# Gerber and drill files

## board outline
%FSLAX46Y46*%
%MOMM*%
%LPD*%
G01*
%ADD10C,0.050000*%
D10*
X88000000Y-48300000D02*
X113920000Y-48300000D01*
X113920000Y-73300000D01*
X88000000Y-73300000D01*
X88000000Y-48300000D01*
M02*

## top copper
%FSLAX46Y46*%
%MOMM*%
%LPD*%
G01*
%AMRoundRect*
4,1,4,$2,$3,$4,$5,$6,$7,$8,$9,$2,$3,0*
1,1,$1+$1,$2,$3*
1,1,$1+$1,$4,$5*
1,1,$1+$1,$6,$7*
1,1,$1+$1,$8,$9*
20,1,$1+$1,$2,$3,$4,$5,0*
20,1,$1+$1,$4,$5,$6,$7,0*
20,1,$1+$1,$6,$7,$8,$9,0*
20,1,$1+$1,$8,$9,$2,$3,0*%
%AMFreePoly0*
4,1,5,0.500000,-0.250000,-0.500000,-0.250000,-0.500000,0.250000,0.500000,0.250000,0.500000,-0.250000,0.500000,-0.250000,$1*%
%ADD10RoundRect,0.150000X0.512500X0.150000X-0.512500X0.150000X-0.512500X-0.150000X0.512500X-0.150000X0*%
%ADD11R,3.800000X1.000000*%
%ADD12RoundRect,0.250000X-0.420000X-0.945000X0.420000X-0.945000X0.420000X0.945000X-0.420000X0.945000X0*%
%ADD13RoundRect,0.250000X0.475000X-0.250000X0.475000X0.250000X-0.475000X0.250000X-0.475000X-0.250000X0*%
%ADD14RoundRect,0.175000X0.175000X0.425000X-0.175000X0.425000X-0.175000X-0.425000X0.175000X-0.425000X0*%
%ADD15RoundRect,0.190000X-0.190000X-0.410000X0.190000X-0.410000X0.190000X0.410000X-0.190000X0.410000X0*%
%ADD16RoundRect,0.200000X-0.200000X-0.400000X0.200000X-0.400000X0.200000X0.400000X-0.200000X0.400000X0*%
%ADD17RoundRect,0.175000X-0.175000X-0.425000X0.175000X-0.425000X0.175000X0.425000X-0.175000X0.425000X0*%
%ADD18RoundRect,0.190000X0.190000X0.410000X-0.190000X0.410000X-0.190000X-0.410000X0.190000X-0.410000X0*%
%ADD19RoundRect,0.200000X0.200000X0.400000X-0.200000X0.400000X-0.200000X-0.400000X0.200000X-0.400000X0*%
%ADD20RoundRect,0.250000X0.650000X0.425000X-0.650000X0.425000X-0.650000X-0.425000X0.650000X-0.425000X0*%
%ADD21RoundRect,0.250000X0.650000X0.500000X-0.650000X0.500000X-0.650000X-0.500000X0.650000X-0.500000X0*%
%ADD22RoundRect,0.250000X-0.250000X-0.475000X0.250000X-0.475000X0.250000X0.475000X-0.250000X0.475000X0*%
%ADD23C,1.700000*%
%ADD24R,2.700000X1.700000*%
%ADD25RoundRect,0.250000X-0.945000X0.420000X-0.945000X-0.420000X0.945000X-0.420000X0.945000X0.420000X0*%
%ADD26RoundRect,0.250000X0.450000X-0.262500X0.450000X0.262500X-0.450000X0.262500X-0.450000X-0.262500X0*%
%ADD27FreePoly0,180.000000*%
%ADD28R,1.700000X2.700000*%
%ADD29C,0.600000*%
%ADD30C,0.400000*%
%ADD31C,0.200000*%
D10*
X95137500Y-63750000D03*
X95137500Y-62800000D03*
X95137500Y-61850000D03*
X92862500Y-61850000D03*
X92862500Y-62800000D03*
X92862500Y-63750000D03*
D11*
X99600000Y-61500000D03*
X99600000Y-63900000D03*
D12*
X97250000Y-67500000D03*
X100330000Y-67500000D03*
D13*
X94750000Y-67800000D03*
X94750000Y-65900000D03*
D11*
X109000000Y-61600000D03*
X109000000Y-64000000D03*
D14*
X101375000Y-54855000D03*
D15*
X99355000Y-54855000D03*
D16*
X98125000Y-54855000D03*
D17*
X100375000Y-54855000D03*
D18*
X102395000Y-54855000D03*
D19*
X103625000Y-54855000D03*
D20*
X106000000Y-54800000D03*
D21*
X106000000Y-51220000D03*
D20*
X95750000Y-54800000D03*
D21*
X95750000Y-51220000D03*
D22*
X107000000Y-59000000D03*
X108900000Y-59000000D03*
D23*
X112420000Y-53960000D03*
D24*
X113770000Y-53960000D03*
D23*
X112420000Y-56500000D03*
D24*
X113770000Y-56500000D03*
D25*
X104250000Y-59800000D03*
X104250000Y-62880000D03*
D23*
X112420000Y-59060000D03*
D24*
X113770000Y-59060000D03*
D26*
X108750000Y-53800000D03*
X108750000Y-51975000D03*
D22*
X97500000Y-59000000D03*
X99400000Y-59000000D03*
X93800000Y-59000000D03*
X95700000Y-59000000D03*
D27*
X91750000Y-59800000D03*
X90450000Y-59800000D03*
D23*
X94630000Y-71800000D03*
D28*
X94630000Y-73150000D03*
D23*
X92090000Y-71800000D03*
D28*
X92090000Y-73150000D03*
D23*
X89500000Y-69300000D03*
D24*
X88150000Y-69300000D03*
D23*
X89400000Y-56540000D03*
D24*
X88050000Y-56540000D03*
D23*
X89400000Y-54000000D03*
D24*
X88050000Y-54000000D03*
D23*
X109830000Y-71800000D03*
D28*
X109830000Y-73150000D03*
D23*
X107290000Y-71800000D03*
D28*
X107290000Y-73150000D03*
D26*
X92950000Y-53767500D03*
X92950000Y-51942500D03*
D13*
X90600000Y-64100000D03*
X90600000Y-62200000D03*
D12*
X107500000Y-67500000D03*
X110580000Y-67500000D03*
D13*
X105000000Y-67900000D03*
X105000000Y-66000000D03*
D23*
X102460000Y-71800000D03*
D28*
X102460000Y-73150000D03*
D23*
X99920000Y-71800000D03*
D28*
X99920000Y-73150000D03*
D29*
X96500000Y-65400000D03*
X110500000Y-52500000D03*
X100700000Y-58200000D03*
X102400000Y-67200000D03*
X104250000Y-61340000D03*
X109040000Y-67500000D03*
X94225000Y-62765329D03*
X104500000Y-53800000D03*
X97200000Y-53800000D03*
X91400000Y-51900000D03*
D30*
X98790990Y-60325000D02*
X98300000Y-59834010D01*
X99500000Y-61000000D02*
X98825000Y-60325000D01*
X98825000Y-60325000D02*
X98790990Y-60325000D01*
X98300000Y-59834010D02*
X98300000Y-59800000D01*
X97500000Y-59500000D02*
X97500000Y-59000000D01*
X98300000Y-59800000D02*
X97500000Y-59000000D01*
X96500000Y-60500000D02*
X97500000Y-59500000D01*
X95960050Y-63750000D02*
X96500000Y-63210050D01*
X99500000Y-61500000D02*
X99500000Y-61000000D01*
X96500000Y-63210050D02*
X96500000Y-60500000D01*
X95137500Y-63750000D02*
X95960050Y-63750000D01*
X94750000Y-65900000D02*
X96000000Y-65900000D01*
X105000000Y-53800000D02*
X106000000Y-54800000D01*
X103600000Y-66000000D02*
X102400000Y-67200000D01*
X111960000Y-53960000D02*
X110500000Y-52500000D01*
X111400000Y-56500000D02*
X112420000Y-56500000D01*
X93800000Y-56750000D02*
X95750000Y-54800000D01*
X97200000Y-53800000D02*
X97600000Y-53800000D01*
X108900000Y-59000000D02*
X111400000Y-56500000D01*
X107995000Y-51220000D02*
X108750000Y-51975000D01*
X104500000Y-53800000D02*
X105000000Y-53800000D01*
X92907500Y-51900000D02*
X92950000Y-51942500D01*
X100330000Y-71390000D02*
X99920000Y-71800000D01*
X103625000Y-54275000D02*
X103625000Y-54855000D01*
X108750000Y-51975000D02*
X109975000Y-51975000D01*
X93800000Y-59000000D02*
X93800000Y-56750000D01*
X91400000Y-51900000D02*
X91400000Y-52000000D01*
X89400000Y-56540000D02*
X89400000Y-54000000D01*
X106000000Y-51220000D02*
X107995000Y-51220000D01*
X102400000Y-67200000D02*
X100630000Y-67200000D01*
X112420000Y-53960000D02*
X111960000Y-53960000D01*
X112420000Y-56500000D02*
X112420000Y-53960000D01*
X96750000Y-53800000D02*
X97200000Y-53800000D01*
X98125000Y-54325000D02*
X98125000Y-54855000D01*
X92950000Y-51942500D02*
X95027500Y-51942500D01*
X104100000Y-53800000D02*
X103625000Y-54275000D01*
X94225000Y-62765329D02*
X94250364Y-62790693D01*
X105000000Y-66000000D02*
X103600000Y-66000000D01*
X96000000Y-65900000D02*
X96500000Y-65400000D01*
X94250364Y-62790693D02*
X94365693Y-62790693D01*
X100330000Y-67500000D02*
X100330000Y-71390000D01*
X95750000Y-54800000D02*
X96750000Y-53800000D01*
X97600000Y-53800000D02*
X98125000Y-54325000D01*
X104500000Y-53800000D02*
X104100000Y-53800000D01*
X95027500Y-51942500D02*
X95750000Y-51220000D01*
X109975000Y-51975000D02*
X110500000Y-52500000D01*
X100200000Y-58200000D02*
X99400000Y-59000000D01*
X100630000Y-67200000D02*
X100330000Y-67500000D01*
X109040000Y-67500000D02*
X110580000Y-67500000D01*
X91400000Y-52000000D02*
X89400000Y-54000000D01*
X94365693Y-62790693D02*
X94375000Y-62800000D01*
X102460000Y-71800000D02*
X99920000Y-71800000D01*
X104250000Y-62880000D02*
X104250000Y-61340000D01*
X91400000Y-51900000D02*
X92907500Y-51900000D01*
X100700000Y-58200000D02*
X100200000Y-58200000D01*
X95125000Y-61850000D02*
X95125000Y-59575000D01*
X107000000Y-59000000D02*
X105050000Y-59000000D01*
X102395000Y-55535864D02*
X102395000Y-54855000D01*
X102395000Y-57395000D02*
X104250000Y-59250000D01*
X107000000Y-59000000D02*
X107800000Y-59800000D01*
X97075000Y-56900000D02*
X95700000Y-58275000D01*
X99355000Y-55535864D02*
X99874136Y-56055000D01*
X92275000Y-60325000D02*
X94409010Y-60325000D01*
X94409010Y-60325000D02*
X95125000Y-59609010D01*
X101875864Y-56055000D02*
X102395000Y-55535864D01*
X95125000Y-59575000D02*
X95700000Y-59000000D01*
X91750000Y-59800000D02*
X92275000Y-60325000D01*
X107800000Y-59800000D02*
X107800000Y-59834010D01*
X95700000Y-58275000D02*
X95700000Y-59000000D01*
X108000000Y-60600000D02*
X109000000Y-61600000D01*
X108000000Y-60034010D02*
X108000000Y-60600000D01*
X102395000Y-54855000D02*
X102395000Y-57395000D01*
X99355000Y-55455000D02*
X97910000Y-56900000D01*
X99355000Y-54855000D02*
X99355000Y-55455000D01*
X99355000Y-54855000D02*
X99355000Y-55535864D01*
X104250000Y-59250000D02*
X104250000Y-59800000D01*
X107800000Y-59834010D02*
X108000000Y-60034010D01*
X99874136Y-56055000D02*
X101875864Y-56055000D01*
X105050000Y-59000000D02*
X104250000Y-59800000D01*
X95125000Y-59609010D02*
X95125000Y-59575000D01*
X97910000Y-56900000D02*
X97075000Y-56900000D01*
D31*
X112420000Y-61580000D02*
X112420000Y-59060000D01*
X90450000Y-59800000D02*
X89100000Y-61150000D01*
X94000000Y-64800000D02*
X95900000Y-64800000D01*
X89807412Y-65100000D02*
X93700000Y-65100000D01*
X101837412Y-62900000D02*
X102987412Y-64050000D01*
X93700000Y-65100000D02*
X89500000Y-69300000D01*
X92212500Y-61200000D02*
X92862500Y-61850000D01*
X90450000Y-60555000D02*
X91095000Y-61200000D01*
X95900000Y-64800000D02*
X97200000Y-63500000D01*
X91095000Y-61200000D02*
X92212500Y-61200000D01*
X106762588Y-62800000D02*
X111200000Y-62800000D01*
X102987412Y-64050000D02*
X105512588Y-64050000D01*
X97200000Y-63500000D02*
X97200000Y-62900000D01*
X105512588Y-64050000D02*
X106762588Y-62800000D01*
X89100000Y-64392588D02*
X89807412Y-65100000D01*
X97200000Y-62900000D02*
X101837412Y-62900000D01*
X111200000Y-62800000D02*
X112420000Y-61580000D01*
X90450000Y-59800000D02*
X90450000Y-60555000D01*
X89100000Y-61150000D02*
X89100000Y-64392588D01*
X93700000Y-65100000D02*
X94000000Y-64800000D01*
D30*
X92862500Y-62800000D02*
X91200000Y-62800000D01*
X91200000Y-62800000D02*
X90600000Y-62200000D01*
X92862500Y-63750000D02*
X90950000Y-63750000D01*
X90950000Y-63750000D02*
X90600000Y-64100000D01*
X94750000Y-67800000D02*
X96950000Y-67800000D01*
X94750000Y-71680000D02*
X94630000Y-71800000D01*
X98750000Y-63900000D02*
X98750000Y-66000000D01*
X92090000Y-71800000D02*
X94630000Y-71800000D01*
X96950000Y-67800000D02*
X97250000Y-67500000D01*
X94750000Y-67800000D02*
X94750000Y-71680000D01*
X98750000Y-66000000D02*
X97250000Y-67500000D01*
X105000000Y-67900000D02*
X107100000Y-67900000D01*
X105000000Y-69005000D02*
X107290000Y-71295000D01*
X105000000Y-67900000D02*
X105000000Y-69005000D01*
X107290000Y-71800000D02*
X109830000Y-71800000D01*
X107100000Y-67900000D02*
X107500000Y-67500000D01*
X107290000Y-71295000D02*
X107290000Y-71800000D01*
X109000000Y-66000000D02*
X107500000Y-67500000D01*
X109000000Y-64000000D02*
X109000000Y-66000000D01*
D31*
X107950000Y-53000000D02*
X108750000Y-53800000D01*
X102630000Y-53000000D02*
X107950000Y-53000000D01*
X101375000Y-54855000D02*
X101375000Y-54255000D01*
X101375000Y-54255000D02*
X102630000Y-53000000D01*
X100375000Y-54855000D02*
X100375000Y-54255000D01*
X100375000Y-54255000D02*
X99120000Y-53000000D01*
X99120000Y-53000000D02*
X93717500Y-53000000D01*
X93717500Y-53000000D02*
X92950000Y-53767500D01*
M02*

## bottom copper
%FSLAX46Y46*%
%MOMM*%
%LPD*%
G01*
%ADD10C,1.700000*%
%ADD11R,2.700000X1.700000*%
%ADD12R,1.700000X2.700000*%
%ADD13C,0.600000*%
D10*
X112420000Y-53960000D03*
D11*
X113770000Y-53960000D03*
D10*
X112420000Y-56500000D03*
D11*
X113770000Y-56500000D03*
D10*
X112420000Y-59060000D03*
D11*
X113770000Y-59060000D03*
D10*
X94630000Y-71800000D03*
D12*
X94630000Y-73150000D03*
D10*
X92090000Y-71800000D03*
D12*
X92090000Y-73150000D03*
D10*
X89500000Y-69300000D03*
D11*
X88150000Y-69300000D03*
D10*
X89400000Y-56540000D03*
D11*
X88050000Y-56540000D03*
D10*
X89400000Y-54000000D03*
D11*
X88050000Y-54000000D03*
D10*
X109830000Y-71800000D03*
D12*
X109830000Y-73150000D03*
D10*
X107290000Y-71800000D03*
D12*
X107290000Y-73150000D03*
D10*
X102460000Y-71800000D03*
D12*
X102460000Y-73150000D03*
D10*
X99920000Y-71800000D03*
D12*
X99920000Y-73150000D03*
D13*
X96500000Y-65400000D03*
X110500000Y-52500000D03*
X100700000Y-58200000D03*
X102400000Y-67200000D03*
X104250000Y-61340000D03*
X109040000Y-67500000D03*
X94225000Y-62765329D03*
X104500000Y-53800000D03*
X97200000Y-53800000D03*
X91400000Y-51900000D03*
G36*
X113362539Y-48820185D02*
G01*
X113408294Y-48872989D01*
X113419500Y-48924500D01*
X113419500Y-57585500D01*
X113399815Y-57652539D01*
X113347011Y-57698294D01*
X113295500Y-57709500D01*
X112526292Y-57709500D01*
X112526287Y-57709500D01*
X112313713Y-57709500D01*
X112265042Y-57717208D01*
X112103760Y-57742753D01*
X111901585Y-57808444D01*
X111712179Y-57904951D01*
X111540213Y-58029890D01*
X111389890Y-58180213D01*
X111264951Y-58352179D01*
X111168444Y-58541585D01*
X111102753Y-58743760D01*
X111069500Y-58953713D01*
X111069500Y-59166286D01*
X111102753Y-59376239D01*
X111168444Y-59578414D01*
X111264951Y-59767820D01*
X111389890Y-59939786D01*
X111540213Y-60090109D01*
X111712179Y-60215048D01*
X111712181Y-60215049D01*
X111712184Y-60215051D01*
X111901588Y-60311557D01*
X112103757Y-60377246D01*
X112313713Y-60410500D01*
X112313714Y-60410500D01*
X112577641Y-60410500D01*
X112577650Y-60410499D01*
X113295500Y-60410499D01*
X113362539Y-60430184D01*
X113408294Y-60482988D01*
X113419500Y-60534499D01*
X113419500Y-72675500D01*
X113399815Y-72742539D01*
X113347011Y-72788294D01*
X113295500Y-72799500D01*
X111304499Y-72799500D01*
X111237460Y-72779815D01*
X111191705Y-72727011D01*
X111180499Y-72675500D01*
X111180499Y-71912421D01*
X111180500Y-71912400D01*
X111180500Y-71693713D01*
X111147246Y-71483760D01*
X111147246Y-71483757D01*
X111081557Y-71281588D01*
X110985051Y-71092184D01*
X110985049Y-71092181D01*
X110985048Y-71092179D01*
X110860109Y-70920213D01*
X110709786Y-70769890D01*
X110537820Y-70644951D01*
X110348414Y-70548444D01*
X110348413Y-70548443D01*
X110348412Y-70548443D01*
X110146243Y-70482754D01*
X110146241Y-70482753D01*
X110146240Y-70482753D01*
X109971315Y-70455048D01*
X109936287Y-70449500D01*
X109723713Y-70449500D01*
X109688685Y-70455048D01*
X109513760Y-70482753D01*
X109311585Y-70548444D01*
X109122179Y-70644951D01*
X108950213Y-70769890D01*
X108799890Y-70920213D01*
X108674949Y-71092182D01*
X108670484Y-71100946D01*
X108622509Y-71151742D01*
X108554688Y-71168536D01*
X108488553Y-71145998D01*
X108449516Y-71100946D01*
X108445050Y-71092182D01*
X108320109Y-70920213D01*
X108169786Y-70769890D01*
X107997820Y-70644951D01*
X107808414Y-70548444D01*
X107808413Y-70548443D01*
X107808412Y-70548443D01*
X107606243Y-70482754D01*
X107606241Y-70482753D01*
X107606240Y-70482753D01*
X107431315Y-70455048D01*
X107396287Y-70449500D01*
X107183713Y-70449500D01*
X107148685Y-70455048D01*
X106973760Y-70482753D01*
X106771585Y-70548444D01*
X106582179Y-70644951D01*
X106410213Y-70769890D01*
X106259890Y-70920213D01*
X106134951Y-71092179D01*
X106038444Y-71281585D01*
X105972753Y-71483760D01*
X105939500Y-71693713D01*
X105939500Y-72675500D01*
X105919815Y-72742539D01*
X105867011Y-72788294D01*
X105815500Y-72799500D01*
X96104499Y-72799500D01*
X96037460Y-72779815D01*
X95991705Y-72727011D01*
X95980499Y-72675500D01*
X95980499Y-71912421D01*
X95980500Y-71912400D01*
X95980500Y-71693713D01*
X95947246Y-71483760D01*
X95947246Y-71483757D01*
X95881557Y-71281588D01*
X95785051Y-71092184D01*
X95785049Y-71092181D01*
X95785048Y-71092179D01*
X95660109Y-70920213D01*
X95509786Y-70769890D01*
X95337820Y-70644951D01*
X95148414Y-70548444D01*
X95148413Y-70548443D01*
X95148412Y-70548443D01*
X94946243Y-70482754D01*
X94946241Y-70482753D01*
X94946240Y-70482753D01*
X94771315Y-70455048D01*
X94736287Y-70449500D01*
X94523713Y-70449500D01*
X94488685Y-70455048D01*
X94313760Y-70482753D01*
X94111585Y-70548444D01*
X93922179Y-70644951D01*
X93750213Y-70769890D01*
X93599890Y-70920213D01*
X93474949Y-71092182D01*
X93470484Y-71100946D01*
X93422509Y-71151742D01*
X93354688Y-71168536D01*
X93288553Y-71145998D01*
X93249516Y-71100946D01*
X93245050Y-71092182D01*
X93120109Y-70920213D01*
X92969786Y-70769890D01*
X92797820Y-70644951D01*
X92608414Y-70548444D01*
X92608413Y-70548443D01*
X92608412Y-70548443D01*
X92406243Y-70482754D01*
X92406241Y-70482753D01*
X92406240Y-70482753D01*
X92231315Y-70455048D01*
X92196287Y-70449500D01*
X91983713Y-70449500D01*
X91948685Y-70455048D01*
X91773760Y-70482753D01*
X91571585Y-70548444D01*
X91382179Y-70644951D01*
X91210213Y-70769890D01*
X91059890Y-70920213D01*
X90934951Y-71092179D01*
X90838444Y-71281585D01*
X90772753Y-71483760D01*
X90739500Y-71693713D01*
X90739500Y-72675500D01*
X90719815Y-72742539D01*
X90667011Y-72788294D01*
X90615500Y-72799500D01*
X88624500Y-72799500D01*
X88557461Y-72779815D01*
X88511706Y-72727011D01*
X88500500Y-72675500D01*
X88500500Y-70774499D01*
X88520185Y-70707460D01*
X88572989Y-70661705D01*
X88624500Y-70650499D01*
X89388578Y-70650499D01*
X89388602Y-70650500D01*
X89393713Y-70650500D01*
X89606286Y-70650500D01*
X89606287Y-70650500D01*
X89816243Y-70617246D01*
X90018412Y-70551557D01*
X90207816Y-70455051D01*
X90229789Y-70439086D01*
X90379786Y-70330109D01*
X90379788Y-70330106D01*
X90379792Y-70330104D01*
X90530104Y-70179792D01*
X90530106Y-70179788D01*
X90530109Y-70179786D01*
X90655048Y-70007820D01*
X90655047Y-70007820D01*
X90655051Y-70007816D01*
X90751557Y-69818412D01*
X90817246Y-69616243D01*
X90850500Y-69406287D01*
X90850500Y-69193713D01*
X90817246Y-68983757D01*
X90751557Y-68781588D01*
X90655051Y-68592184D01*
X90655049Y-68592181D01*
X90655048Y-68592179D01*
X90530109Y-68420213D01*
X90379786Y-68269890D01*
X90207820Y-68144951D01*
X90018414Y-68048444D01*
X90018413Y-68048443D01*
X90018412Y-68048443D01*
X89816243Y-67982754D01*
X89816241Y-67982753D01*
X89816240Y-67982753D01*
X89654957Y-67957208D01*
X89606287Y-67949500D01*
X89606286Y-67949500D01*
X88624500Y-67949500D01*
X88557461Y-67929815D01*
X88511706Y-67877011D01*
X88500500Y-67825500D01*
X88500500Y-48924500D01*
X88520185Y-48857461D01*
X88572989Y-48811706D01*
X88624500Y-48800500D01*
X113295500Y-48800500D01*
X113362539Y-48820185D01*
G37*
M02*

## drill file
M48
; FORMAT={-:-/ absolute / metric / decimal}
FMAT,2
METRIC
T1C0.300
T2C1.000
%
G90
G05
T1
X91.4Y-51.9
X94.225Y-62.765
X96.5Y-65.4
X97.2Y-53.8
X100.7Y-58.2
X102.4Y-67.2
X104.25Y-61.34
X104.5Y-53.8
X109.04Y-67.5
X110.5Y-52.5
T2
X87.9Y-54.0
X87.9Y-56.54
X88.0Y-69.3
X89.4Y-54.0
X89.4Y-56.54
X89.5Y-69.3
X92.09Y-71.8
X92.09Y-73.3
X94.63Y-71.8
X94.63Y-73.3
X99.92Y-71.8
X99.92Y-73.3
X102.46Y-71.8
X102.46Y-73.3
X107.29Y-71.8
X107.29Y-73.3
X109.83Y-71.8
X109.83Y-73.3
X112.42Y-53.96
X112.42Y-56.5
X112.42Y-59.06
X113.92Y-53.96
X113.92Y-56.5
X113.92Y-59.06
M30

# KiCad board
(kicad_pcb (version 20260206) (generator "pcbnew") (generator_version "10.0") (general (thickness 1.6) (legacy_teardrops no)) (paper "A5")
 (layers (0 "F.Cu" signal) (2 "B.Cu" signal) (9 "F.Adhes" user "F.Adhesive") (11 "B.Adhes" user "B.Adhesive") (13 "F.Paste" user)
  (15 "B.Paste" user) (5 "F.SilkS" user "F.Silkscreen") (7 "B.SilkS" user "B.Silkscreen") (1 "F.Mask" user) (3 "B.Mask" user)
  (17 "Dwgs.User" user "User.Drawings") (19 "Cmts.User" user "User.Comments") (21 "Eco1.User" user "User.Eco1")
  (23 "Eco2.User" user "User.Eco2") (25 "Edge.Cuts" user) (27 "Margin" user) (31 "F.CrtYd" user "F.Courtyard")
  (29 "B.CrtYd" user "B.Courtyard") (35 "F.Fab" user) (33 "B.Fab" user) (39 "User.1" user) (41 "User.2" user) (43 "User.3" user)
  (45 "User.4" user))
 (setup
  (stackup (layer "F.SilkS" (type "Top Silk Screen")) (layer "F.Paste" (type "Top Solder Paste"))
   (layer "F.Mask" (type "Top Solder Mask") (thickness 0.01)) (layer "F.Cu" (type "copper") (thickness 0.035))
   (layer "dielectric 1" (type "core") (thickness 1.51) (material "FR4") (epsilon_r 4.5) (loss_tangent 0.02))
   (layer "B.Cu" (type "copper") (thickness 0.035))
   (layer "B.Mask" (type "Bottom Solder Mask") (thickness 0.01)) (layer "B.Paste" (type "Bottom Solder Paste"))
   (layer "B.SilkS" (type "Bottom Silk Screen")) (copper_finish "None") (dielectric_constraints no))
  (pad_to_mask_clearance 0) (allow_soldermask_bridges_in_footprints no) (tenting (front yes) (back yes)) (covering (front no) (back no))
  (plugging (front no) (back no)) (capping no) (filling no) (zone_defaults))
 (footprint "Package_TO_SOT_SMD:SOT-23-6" (layer "F.Cu") (at 94 62.8 180)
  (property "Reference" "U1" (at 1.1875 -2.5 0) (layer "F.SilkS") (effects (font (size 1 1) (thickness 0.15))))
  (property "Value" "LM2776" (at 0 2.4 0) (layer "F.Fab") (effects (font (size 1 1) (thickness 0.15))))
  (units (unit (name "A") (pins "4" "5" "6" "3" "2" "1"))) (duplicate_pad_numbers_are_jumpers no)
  (pad "1" smd roundrect (at -1.1375 -0.95 180) (size 1.325 0.6) (layers "F.Cu" "F.Mask" "F.Paste") (roundrect_rratio 0.25) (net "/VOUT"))
  (pad "2" smd roundrect (at -1.1375 0 180) (size 1.325 0.6) (layers "F.Cu" "F.Mask" "F.Paste") (roundrect_rratio 0.25) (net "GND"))
  (pad "3" smd roundrect (at -1.1375 0.95 180) (size 1.325 0.6) (layers "F.Cu" "F.Mask" "F.Paste") (roundrect_rratio 0.25) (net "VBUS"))
  (pad "4" smd roundrect (at 1.1375 0.95 180) (size 1.325 0.6) (layers "F.Cu" "F.Mask" "F.Paste") (roundrect_rratio 0.25) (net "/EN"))
  (pad "5" smd roundrect (at 1.1375 0 180) (size 1.325 0.6) (layers "F.Cu" "F.Mask" "F.Paste") (roundrect_rratio 0.25) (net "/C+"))
  (pad "6" smd roundrect (at 1.1375 -0.95 180) (size 1.325 0.6) (layers "F.Cu" "F.Mask" "F.Paste") (roundrect_rratio 0.25) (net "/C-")))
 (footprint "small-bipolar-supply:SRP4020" (layer "F.Cu") (at 99.6 62.7)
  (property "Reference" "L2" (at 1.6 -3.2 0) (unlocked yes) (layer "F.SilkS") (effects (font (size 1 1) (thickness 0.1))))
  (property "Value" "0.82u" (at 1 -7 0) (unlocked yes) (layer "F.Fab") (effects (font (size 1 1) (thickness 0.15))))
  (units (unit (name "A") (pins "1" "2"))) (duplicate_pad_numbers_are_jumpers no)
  (pad "1" smd rect (at 0 -1.2) (size 3.8 1) (layers "F.Cu" "F.Mask" "F.Paste") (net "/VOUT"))
  (pad "2" smd rect (at 0 1.2) (size 3.8 1) (layers "F.Cu" "F.Mask" "F.Paste") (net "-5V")))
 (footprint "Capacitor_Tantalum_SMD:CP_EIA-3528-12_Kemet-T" (layer "F.Cu") (at 98.79 67.5)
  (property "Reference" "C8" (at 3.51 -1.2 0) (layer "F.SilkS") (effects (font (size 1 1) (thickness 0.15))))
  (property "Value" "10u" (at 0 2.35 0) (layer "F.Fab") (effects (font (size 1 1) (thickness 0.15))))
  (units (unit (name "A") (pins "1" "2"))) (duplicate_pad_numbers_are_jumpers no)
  (pad "1" smd roundrect (at -1.54 0) (size 1.34 2.39) (layers "F.Cu" "F.Mask" "F.Paste") (roundrect_rratio 0.186567) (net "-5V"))
  (pad "2" smd roundrect (at 1.54 0) (size 1.34 2.39) (layers "F.Cu" "F.Mask" "F.Paste") (roundrect_rratio 0.186567) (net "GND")))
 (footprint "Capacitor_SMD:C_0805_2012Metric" (layer "F.Cu") (at 94.75 66.85 90)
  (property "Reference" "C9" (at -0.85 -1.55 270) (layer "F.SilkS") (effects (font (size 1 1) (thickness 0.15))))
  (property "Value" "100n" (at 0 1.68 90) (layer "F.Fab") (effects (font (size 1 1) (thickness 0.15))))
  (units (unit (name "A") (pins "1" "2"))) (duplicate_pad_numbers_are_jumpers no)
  (pad "1" smd roundrect (at -0.95 0 90) (size 1 1.45) (layers "F.Cu" "F.Mask" "F.Paste") (roundrect_rratio 0.25) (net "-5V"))
  (pad "2" smd roundrect (at 0.95 0 90) (size 1 1.45) (layers "F.Cu" "F.Mask" "F.Paste") (roundrect_rratio 0.25) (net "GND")))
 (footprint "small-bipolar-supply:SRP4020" (layer "F.Cu") (at 109 62.8)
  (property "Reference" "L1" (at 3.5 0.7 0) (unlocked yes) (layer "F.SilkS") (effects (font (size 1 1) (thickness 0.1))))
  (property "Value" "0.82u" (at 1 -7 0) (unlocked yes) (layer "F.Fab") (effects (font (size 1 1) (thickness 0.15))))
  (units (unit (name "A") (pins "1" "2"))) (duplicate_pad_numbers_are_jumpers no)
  (pad "1" smd rect (at 0 -1.2) (size 3.8 1) (layers "F.Cu" "F.Mask" "F.Paste") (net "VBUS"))
  (pad "2" smd rect (at 0 1.2) (size 3.8 1) (layers "F.Cu" "F.Mask" "F.Paste") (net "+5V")))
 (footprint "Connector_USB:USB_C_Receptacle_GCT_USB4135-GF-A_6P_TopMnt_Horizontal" (layer "F.Cu") (at 100.875 51.8225 180)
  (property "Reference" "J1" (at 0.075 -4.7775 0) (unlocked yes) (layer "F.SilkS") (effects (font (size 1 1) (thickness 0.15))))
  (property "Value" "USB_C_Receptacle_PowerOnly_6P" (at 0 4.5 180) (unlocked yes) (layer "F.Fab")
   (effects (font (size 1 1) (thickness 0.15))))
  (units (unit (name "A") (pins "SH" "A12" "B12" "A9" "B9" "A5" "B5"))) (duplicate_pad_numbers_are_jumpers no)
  (pad "A5" smd roundrect (at -0.5 -3.0325 180) (size 0.7 1.2) (layers "F.Cu" "F.Mask" "F.Paste") (roundrect_rratio 0.25)
   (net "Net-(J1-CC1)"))
  (pad "A9" smd roundrect (at 1.52 -3.0325) (size 0.76 1.2) (layers "F.Cu" "F.Mask" "F.Paste") (roundrect_rratio 0.25) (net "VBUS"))
  (pad "A12" smd roundrect (at 2.75 -3.0325) (size 0.8 1.2) (layers "F.Cu" "F.Mask" "F.Paste") (roundrect_rratio 0.25) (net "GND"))
  (pad "B5" smd roundrect (at 0.5 -3.0325) (size 0.7 1.2) (layers "F.Cu" "F.Mask" "F.Paste") (roundrect_rratio 0.25) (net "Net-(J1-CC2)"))
  (pad "B9" smd roundrect (at -1.52 -3.0325 180) (size 0.76 1.2) (layers "F.Cu" "F.Mask" "F.Paste") (roundrect_rratio 0.25) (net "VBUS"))
  (pad "B12" smd roundrect (at -2.75 -3.0325 180) (size 0.8 1.2) (layers "F.Cu" "F.Mask" "F.Paste") (roundrect_rratio 0.25) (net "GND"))
  (pad "SH" smd roundrect (at -5.125 -2.9775 180) (size 1.8 1.35) (layers "F.Cu" "F.Mask" "F.Paste") (roundrect_rratio 0.1851851852)
   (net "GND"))
  (pad "SH" smd roundrect (at -5.125 0.6025 180) (size 1.8 1.5) (layers "F.Cu" "F.Mask" "F.Paste") (roundrect_rratio 0.1666666667)
   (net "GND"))
  (pad "SH" smd roundrect (at 5.125 -2.9775 180) (size 1.8 1.35) (layers "F.Cu" "F.Mask" "F.Paste") (roundrect_rratio 0.1851851852)
   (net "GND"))
  (pad "SH" smd roundrect (at 5.125 0.6025 180) (size 1.8 1.5) (layers "F.Cu" "F.Mask" "F.Paste") (roundrect_rratio 0.1666666667)
   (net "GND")))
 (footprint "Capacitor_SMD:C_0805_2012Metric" (layer "F.Cu") (at 107.95 59)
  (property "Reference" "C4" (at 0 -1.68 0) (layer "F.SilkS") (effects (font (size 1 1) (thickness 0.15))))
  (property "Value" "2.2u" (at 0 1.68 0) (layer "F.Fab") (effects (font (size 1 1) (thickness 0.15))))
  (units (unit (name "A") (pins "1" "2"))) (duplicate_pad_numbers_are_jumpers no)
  (pad "1" smd roundrect (at -0.95 0) (size 1 1.45) (layers "F.Cu" "F.Mask" "F.Paste") (roundrect_rratio 0.25) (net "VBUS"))
  (pad "2" smd roundrect (at 0.95 0) (size 1 1.45) (layers "F.Cu" "F.Mask" "F.Paste") (roundrect_rratio 0.25) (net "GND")))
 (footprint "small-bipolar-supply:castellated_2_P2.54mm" (layer "F.Cu") (at 113.92 54)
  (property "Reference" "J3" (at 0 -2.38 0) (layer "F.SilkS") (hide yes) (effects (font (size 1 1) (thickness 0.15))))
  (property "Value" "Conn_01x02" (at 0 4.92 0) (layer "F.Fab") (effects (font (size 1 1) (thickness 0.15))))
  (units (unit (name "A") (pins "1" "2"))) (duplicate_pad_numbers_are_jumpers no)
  (pad "1" thru_hole circle (at -1.5 -0.04) (size 1.7 1.7) (drill 1) (layers "*.Cu" "*.Mask") (remove_unused_layers no) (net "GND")
   (zone_connect 2))
  (pad "1" thru_hole rect (at 0 -0.04) (size 2.7 1.7) (drill 1 (offset -0.15 0)) (layers "*.Cu" "*.Mask") (remove_unused_layers no)
   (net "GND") (zone_connect 2))
  (pad "2" thru_hole circle (at -1.5 2.5) (size 1.7 1.7) (drill 1) (layers "*.Cu" "*.Mask") (remove_unused_layers no) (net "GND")
   (zone_connect 2))
  (pad "2" thru_hole rect (at 0 2.5) (size 2.7 1.7) (drill 1 (offset -0.15 0)) (layers "*.Cu" "*.Mask") (remove_unused_layers no)
   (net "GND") (zone_connect 2)))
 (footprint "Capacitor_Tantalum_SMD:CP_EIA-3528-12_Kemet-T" (layer "F.Cu") (at 104.25 61.34 -90)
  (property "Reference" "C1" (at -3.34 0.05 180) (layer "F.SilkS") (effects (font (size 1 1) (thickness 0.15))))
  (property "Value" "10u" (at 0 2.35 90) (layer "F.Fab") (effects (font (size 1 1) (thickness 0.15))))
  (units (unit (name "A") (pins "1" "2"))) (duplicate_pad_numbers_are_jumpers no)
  (pad "1" smd roundrect (at -1.54 0 270) (size 1.34 2.39) (layers "F.Cu" "F.Mask" "F.Paste") (roundrect_rratio 0.186567) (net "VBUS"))
  (pad "2" smd roundrect (at 1.54 0 270) (size 1.34 2.39) (layers "F.Cu" "F.Mask" "F.Paste") (roundrect_rratio 0.186567) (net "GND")))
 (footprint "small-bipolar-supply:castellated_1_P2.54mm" (layer "F.Cu") (at 113.92 59.1)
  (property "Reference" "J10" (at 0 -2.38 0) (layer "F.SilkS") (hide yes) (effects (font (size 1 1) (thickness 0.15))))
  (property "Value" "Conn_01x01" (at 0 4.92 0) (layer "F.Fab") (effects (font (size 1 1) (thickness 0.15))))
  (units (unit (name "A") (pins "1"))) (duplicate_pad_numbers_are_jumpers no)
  (pad "1" thru_hole circle (at -1.5 -0.04) (size 1.7 1.7) (drill 1) (layers "*.Cu" "*.Mask") (remove_unused_layers no) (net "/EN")
   (zone_connect 2))
  (pad "1" thru_hole rect (at 0 -0.04) (size 2.7 1.7) (drill 1 (offset -0.15 0)) (layers "*.Cu" "*.Mask") (remove_unused_layers no)
   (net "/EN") (zone_connect 2)))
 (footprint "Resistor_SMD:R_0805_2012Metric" (layer "F.Cu") (at 108.75 52.8875 90)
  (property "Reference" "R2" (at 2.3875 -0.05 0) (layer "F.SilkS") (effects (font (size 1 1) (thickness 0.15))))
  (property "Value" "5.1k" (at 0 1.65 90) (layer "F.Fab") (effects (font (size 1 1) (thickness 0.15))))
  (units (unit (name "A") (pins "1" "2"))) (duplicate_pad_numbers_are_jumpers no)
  (pad "1" smd roundrect (at -0.9125 0 90) (size 1.025 1.4) (layers "F.Cu" "F.Mask" "F.Paste") (roundrect_rratio 0.243902)
   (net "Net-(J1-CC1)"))
  (pad "2" smd roundrect (at 0.9125 0 90) (size 1.025 1.4) (layers "F.Cu" "F.Mask" "F.Paste") (roundrect_rratio 0.243902) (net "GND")))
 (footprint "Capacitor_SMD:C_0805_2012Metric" (layer "F.Cu") (at 98.45 59)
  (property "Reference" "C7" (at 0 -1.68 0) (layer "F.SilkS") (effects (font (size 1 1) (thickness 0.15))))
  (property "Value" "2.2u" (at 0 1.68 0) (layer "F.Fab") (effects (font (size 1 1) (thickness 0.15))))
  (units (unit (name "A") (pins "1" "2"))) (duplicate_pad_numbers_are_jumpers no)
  (pad "1" smd roundrect (at -0.95 0) (size 1 1.45) (layers "F.Cu" "F.Mask" "F.Paste") (roundrect_rratio 0.25) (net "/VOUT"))
  (pad "2" smd roundrect (at 0.95 0) (size 1 1.45) (layers "F.Cu" "F.Mask" "F.Paste") (roundrect_rratio 0.25) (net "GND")))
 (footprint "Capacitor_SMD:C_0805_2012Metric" (layer "F.Cu") (at 94.75 59)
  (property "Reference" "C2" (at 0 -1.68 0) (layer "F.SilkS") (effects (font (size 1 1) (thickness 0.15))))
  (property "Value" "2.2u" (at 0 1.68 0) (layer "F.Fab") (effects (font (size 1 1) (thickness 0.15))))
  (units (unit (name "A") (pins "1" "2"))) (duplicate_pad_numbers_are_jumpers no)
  (pad "1" smd roundrect (at -0.95 0) (size 1 1.45) (layers "F.Cu" "F.Mask" "F.Paste") (roundrect_rratio 0.25) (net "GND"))
  (pad "2" smd roundrect (at 0.95 0) (size 1 1.45) (layers "F.Cu" "F.Mask" "F.Paste") (roundrect_rratio 0.25) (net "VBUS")))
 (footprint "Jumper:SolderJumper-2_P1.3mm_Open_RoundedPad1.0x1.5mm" (layer "F.Cu") (at 91.1 59.8 180)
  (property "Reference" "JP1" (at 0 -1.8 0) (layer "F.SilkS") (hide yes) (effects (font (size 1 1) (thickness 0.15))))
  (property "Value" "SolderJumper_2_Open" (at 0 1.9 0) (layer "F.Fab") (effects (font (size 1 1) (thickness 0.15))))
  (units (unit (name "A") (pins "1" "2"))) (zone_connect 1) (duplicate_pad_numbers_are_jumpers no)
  (pad "1" smd custom (at -0.65 0 180) (size 1 0.5) (layers "F.Cu" "F.Mask") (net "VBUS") (zone_connect 2) (thermal_bridge_angle 45)
   (options (clearance outline) (anchor rect)) (primitives))
  (pad "2" smd custom (at 0.65 0 180) (size 1 0.5) (layers "F.Cu" "F.Mask") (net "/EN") (zone_connect 2) (thermal_bridge_angle 45)
   (options (clearance outline) (anchor rect)) (primitives)))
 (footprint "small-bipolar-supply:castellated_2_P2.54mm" (layer "F.Cu") (at 94.59 73.3 -90)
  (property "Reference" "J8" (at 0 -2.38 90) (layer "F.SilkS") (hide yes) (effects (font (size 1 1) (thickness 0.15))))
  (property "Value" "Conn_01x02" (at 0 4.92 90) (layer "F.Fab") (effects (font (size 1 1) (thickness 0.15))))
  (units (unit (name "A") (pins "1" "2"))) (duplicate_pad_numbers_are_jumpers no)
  (pad "1" thru_hole circle (at -1.5 -0.04 270) (size 1.7 1.7) (drill 1) (layers "*.Cu" "*.Mask") (remove_unused_layers no) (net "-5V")
   (zone_connect 2))
  (pad "1" thru_hole rect (at 0 -0.04 270) (size 2.7 1.7) (drill 1 (offset -0.15 0)) (layers "*.Cu" "*.Mask") (remove_unused_layers no)
   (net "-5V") (zone_connect 2))
  (pad "2" thru_hole circle (at -1.5 2.5 270) (size 1.7 1.7) (drill 1) (layers "*.Cu" "*.Mask") (remove_unused_layers no) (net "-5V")
   (zone_connect 2))
  (pad "2" thru_hole rect (at 0 2.5 270) (size 2.7 1.7) (drill 1 (offset -0.15 0)) (layers "*.Cu" "*.Mask") (remove_unused_layers no)
   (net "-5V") (zone_connect 2)))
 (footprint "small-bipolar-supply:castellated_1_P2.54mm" (layer "F.Cu") (at 88 69.26 180)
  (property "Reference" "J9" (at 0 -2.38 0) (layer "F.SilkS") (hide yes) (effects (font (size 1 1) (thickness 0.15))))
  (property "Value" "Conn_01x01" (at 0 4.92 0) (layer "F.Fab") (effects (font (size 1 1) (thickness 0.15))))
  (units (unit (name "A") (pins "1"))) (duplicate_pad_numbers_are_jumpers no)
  (pad "1" thru_hole circle (at -1.5 -0.04 180) (size 1.7 1.7) (drill 1) (layers "*.Cu" "*.Mask") (remove_unused_layers no) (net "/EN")
   (zone_connect 2))
  (pad "1" thru_hole rect (at 0 -0.04 180) (size 2.7 1.7) (drill 1 (offset -0.15 0)) (layers "*.Cu" "*.Mask") (remove_unused_layers no)
   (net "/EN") (zone_connect 2)))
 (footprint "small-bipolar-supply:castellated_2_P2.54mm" (layer "F.Cu") (at 87.9 56.5 180)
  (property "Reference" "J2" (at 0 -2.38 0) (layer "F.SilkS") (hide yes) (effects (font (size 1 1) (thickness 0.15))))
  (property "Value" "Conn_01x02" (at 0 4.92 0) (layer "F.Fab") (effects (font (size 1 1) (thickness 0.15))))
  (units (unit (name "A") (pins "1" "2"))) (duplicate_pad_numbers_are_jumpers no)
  (pad "1" thru_hole circle (at -1.5 -0.04 180) (size 1.7 1.7) (drill 1) (layers "*.Cu" "*.Mask") (remove_unused_layers no) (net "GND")
   (zone_connect 2))
  (pad "1" thru_hole rect (at 0 -0.04 180) (size 2.7 1.7) (drill 1 (offset -0.15 0)) (layers "*.Cu" "*.Mask") (remove_unused_layers no)
   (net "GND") (zone_connect 2))
  (pad "2" thru_hole circle (at -1.5 2.5 180) (size 1.7 1.7) (drill 1) (layers "*.Cu" "*.Mask") (remove_unused_layers no) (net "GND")
   (zone_connect 2))
  (pad "2" thru_hole rect (at 0 2.5 180) (size 2.7 1.7) (drill 1 (offset -0.15 0)) (layers "*.Cu" "*.Mask") (remove_unused_layers no)
   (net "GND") (zone_connect 2)))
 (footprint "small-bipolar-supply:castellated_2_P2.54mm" (layer "F.Cu") (at 109.79 73.3 -90)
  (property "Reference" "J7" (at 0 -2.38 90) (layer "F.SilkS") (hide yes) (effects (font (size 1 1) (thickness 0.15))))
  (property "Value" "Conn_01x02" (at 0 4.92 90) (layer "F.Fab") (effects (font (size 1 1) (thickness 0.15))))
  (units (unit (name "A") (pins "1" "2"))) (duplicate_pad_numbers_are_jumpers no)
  (pad "1" thru_hole circle (at -1.5 -0.04 270) (size 1.7 1.7) (drill 1) (layers "*.Cu" "*.Mask") (remove_unused_layers no) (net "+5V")
   (zone_connect 2))
  (pad "1" thru_hole rect (at 0 -0.04 270) (size 2.7 1.7) (drill 1 (offset -0.15 0)) (layers "*.Cu" "*.Mask") (remove_unused_layers no)
   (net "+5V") (zone_connect 2))
  (pad "2" thru_hole circle (at -1.5 2.5 270) (size 1.7 1.7) (drill 1) (layers "*.Cu" "*.Mask") (remove_unused_layers no) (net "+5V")
   (zone_connect 2))
  (pad "2" thru_hole rect (at 0 2.5 270) (size 2.7 1.7) (drill 1 (offset -0.15 0)) (layers "*.Cu" "*.Mask") (remove_unused_layers no)
   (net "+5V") (zone_connect 2)))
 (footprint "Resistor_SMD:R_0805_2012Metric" (layer "F.Cu") (at 92.95 52.855 90)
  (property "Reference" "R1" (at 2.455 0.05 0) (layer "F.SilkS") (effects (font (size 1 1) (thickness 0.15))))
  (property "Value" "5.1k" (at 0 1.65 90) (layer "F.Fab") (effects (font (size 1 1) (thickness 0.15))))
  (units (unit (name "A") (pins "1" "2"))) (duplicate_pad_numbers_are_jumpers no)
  (pad "1" smd roundrect (at -0.9125 0 90) (size 1.025 1.4) (layers "F.Cu" "F.Mask" "F.Paste") (roundrect_rratio 0.243902)
   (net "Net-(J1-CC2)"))
  (pad "2" smd roundrect (at 0.9125 0 90) (size 1.025 1.4) (layers "F.Cu" "F.Mask" "F.Paste") (roundrect_rratio 0.243902) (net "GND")))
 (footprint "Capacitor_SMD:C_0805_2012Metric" (layer "F.Cu") (at 90.6 63.15 90)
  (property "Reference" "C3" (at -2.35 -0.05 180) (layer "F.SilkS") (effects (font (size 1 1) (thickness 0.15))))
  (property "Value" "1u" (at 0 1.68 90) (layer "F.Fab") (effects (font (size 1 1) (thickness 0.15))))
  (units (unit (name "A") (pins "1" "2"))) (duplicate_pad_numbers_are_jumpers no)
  (pad "1" smd roundrect (at -0.95 0 90) (size 1 1.45) (layers "F.Cu" "F.Mask" "F.Paste") (roundrect_rratio 0.25) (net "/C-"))
  (pad "2" smd roundrect (at 0.95 0 90) (size 1 1.45) (layers "F.Cu" "F.Mask" "F.Paste") (roundrect_rratio 0.25) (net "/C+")))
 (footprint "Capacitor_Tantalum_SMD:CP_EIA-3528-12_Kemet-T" (layer "F.Cu") (at 109.04 67.5)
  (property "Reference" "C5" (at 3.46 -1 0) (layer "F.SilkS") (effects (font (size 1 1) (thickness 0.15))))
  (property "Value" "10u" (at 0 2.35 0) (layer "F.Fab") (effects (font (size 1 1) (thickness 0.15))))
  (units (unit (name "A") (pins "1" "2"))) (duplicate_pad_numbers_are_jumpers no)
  (pad "1" smd roundrect (at -1.54 0) (size 1.34 2.39) (layers "F.Cu" "F.Mask" "F.Paste") (roundrect_rratio 0.186567) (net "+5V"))
  (pad "2" smd roundrect (at 1.54 0) (size 1.34 2.39) (layers "F.Cu" "F.Mask" "F.Paste") (roundrect_rratio 0.186567) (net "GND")))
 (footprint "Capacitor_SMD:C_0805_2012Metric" (layer "F.Cu") (at 105 66.95 90)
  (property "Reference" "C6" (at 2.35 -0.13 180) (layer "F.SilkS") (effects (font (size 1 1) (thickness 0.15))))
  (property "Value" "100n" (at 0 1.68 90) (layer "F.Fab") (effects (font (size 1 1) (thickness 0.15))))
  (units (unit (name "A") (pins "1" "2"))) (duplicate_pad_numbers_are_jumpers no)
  (pad "1" smd roundrect (at -0.95 0 90) (size 1 1.45) (layers "F.Cu" "F.Mask" "F.Paste") (roundrect_rratio 0.25) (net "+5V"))
  (pad "2" smd roundrect (at 0.95 0 90) (size 1 1.45) (layers "F.Cu" "F.Mask" "F.Paste") (roundrect_rratio 0.25) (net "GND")))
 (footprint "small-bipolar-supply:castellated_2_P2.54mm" (layer "F.Cu") (at 102.42 73.3 -90)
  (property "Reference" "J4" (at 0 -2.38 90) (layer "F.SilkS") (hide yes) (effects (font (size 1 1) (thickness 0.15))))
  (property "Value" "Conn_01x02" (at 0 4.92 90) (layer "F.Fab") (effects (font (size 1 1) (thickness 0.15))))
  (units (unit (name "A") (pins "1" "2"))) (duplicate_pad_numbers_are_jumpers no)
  (pad "1" thru_hole circle (at -1.5 -0.04 270) (size 1.7 1.7) (drill 1) (layers "*.Cu" "*.Mask") (remove_unused_layers no) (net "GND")
   (zone_connect 2))
  (pad "1" thru_hole rect (at 0 -0.04 270) (size 2.7 1.7) (drill 1 (offset -0.15 0)) (layers "*.Cu" "*.Mask") (remove_unused_layers no)
   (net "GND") (zone_connect 2))
  (pad "2" thru_hole circle (at -1.5 2.5 270) (size 1.7 1.7) (drill 1) (layers "*.Cu" "*.Mask") (remove_unused_layers no) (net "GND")
   (zone_connect 2))
  (pad "2" thru_hole rect (at 0 2.5 270) (size 2.7 1.7) (drill 1 (offset -0.15 0)) (layers "*.Cu" "*.Mask") (remove_unused_layers no)
   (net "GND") (zone_connect 2)))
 (gr_rect (start 88 48.3) (end 113.92 73.3) (stroke (width 0.05) (type solid)) (fill no) (layer "Edge.Cuts"))
 (segment (start 98.79099 60.325) (end 98.3 59.83401) (width 0.4) (layer "F.Cu") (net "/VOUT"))
 (segment (start 99.5 61) (end 98.825 60.325) (width 0.4) (layer "F.Cu") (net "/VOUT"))
 (segment (start 98.825 60.325) (end 98.79099 60.325) (width 0.4) (layer "F.Cu") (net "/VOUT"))
 (segment (start 98.3 59.83401) (end 98.3 59.8) (width 0.4) (layer "F.Cu") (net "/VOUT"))
 (segment (start 97.5 59.5) (end 97.5 59) (width 0.4) (layer "F.Cu") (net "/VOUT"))
 (segment (start 98.3 59.8) (end 97.5 59) (width 0.4) (layer "F.Cu") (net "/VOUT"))
 (segment (start 96.5 60.5) (end 97.5 59.5) (width 0.4) (layer "F.Cu") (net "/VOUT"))
 (segment (start 95.96005 63.75) (end 96.5 63.21005) (width 0.4) (layer "F.Cu") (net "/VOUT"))
 (segment (start 99.5 61.5) (end 99.5 61) (width 0.4) (layer "F.Cu") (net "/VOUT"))
 (segment (start 96.5 63.21005) (end 96.5 60.5) (width 0.4) (layer "F.Cu") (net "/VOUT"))
 (segment (start 95.1375 63.75) (end 95.96005 63.75) (width 0.4) (layer "F.Cu") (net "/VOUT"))
 (segment (start 94.75 65.9) (end 96 65.9) (width 0.4) (layer "F.Cu") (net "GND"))
 (segment (start 105 53.8) (end 106 54.8) (width 0.4) (layer "F.Cu") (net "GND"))
 (segment (start 103.6 66) (end 102.4 67.2) (width 0.4) (layer "F.Cu") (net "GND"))
 (segment (start 111.96 53.96) (end 110.5 52.5) (width 0.4) (layer "F.Cu") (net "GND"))
 (segment (start 111.4 56.5) (end 112.42 56.5) (width 0.4) (layer "F.Cu") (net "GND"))
 (segment (start 93.8 56.75) (end 95.75 54.8) (width 0.4) (layer "F.Cu") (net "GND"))
 (segment (start 97.2 53.8) (end 97.6 53.8) (width 0.4) (layer "F.Cu") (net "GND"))
 (segment (start 108.9 59) (end 111.4 56.5) (width 0.4) (layer "F.Cu") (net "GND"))
 (segment (start 107.995 51.22) (end 108.75 51.975) (width 0.4) (layer "F.Cu") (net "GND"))
 (segment (start 104.5 53.8) (end 105 53.8) (width 0.4) (layer "F.Cu") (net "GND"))
 (segment (start 92.9075 51.9) (end 92.95 51.9425) (width 0.4) (layer "F.Cu") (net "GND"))
 (segment (start 100.33 71.39) (end 99.92 71.8) (width 0.4) (layer "F.Cu") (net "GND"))
 (segment (start 103.625 54.275) (end 103.625 54.855) (width 0.4) (layer "F.Cu") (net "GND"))
 (segment (start 108.75 51.975) (end 109.975 51.975) (width 0.4) (layer "F.Cu") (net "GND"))
 (segment (start 93.8 59) (end 93.8 56.75) (width 0.4) (layer "F.Cu") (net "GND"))
 (segment (start 91.4 51.9) (end 91.4 52) (width 0.4) (layer "F.Cu") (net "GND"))
 (segment (start 89.4 56.54) (end 89.4 54) (width 0.4) (layer "F.Cu") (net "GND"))
 (segment (start 106 51.22) (end 107.995 51.22) (width 0.4) (layer "F.Cu") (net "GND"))
 (segment (start 102.4 67.2) (end 100.63 67.2) (width 0.4) (layer "F.Cu") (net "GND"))
 (segment (start 112.42 53.96) (end 111.96 53.96) (width 0.4) (layer "F.Cu") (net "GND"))
 (segment (start 112.42 56.5) (end 112.42 53.96) (width 0.4) (layer "F.Cu") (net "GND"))
 (segment (start 96.75 53.8) (end 97.2 53.8) (width 0.4) (layer "F.Cu") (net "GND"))
 (segment (start 98.125 54.325) (end 98.125 54.855) (width 0.4) (layer "F.Cu") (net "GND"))
 (segment (start 92.95 51.9425) (end 95.0275 51.9425) (width 0.4) (layer "F.Cu") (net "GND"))
 (segment (start 104.1 53.8) (end 103.625 54.275) (width 0.4) (layer "F.Cu") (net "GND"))
 (segment (start 94.225 62.765329) (end 94.250364 62.790693) (width 0.4) (layer "F.Cu") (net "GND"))
 (segment (start 105 66) (end 103.6 66) (width 0.4) (layer "F.Cu") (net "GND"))
 (segment (start 96 65.9) (end 96.5 65.4) (width 0.4) (layer "F.Cu") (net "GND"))
 (segment (start 94.250364 62.790693) (end 94.365693 62.790693) (width 0.4) (layer "F.Cu") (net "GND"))
 (segment (start 100.33 67.5) (end 100.33 71.39) (width 0.4) (layer "F.Cu") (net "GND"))
 (segment (start 95.75 54.8) (end 96.75 53.8) (width 0.4) (layer "F.Cu") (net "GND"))
 (segment (start 97.6 53.8) (end 98.125 54.325) (width 0.4) (layer "F.Cu") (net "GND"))
 (segment (start 104.5 53.8) (end 104.1 53.8) (width 0.4) (layer "F.Cu") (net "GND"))
 (segment (start 95.0275 51.9425) (end 95.75 51.22) (width 0.4) (layer "F.Cu") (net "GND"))
 (segment (start 109.975 51.975) (end 110.5 52.5) (width 0.4) (layer "F.Cu") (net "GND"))
 (segment (start 100.2 58.2) (end 99.4 59) (width 0.4) (layer "F.Cu") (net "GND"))
 (segment (start 100.63 67.2) (end 100.33 67.5) (width 0.4) (layer "F.Cu") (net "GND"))
 (segment (start 109.04 67.5) (end 110.58 67.5) (width 0.4) (layer "F.Cu") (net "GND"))
 (segment (start 91.4 52) (end 89.4 54) (width 0.4) (layer "F.Cu") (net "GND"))
 (segment (start 94.365693 62.790693) (end 94.375 62.8) (width 0.4) (layer "F.Cu") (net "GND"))
 (segment (start 102.46 71.8) (end 99.92 71.8) (width 0.4) (layer "F.Cu") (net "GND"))
 (segment (start 104.25 62.88) (end 104.25 61.34) (width 0.4) (layer "F.Cu") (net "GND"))
 (segment (start 91.4 51.9) (end 92.9075 51.9) (width 0.4) (layer "F.Cu") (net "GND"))
 (segment (start 100.7 58.2) (end 100.2 58.2) (width 0.4) (layer "F.Cu") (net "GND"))
 (via (at 96.5 65.4) (size 0.6) (drill 0.3) (layers "F.Cu" "B.Cu") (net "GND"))
 (via (at 110.5 52.5) (size 0.6) (drill 0.3) (layers "F.Cu" "B.Cu") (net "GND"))
 (via (at 100.7 58.2) (size 0.6) (drill 0.3) (layers "F.Cu" "B.Cu") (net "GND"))
 (via (at 102.4 67.2) (size 0.6) (drill 0.3) (layers "F.Cu" "B.Cu") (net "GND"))
 (via (at 104.25 61.34) (size 0.6) (drill 0.3) (layers "F.Cu" "B.Cu") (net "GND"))
 (via (at 109.04 67.5) (size 0.6) (drill 0.3) (layers "F.Cu" "B.Cu") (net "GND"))
 (via (at 94.225 62.765329) (size 0.6) (drill 0.3) (layers "F.Cu" "B.Cu") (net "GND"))
 (via (at 104.5 53.8) (size 0.6) (drill 0.3) (layers "F.Cu" "B.Cu") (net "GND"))
 (via (at 97.2 53.8) (size 0.6) (drill 0.3) (layers "F.Cu" "B.Cu") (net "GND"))
 (via (at 91.4 51.9) (size 0.6) (drill 0.3) (layers "F.Cu" "B.Cu") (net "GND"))
 (segment (start 95.125 61.85) (end 95.125 59.575) (width 0.4) (layer "F.Cu") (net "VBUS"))
 (segment (start 107 59) (end 105.05 59) (width 0.4) (layer "F.Cu") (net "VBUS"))
 (segment (start 102.395 55.535864) (end 102.395 54.855) (width 0.4) (layer "F.Cu") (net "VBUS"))
 (segment (start 102.395 57.395) (end 104.25 59.25) (width 0.4) (layer "F.Cu") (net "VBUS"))
 (segment (start 107 59) (end 107.8 59.8) (width 0.4) (layer "F.Cu") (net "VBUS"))
 (segment (start 97.075 56.9) (end 95.7 58.275) (width 0.4) (layer "F.Cu") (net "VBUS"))
 (segment (start 99.355 55.535864) (end 99.874136 56.055) (width 0.4) (layer "F.Cu") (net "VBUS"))
 (segment (start 92.275 60.325) (end 94.40901 60.325) (width 0.4) (layer "F.Cu") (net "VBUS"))
 (segment (start 94.40901 60.325) (end 95.125 59.60901) (width 0.4) (layer "F.Cu") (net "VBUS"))
 (segment (start 101.875864 56.055) (end 102.395 55.535864) (width 0.4) (layer "F.Cu") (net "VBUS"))
 (segment (start 95.125 59.575) (end 95.7 59) (width 0.4) (layer "F.Cu") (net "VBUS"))
 (segment (start 91.75 59.8) (end 92.275 60.325) (width 0.4) (layer "F.Cu") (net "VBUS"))
 (segment (start 107.8 59.8) (end 107.8 59.83401) (width 0.4) (layer "F.Cu") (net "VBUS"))
 (segment (start 95.7 58.275) (end 95.7 59) (width 0.4) (layer "F.Cu") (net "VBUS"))
 (segment (start 108 60.6) (end 109 61.6) (width 0.4) (layer "F.Cu") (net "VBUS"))
 (segment (start 108 60.03401) (end 108 60.6) (width 0.4) (layer "F.Cu") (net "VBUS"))
 (segment (start 102.395 54.855) (end 102.395 57.395) (width 0.4) (layer "F.Cu") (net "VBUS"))
 (segment (start 99.355 55.455) (end 97.91 56.9) (width 0.4) (layer "F.Cu") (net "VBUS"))
 (segment (start 99.355 54.855) (end 99.355 55.455) (width 0.4) (layer "F.Cu") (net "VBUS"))
 (segment (start 99.355 54.855) (end 99.355 55.535864) (width 0.4) (layer "F.Cu") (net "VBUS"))
 (segment (start 104.25 59.25) (end 104.25 59.8) (width 0.4) (layer "F.Cu") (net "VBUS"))
 (segment (start 107.8 59.83401) (end 108 60.03401) (width 0.4) (layer "F.Cu") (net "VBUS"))
 (segment (start 99.874136 56.055) (end 101.875864 56.055) (width 0.4) (layer "F.Cu") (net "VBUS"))
 (segment (start 105.05 59) (end 104.25 59.8) (width 0.4) (layer "F.Cu") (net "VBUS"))
 (segment (start 95.125 59.60901) (end 95.125 59.575) (width 0.4) (layer "F.Cu") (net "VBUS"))
 (segment (start 97.91 56.9) (end 97.075 56.9) (width 0.4) (layer "F.Cu") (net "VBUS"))
 (segment (start 112.42 61.58) (end 112.42 59.06) (width 0.2) (layer "F.Cu") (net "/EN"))
 (segment (start 90.45 59.8) (end 89.1 61.15) (width 0.2) (layer "F.Cu") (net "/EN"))
 (segment (start 94 64.8) (end 95.9 64.8) (width 0.2) (layer "F.Cu") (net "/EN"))
 (segment (start 89.807412 65.1) (end 93.7 65.1) (width 0.2) (layer "F.Cu") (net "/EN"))
 (segment (start 101.837412 62.9) (end 102.987412 64.05) (width 0.2) (layer "F.Cu") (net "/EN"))
 (segment (start 93.7 65.1) (end 89.5 69.3) (width 0.2) (layer "F.Cu") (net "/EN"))
 (segment (start 92.2125 61.2) (end 92.8625 61.85) (width 0.2) (layer "F.Cu") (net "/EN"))
 (segment (start 90.45 60.555) (end 91.095 61.2) (width 0.2) (layer "F.Cu") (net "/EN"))
 (segment (start 95.9 64.8) (end 97.2 63.5) (width 0.2) (layer "F.Cu") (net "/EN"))
 (segment (start 91.095 61.2) (end 92.2125 61.2) (width 0.2) (layer "F.Cu") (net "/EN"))
 (segment (start 106.762588 62.8) (end 111.2 62.8) (width 0.2) (layer "F.Cu") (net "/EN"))
 (segment (start 102.987412 64.05) (end 105.512588 64.05) (width 0.2) (layer "F.Cu") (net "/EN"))
 (segment (start 97.2 63.5) (end 97.2 62.9) (width 0.2) (layer "F.Cu") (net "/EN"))
 (segment (start 105.512588 64.05) (end 106.762588 62.8) (width 0.2) (layer "F.Cu") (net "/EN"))
 (segment (start 89.1 64.392588) (end 89.807412 65.1) (width 0.2) (layer "F.Cu") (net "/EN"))
 (segment (start 97.2 62.9) (end 101.837412 62.9) (width 0.2) (layer "F.Cu") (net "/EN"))
 (segment (start 111.2 62.8) (end 112.42 61.58) (width 0.2) (layer "F.Cu") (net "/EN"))
 (segment (start 90.45 59.8) (end 90.45 60.555) (width 0.2) (layer "F.Cu") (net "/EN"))
 (segment (start 89.1 61.15) (end 89.1 64.392588) (width 0.2) (layer "F.Cu") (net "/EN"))
 (segment (start 93.7 65.1) (end 94 64.8) (width 0.2) (layer "F.Cu") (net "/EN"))
 (segment (start 92.8625 62.8) (end 91.2 62.8) (width 0.4) (layer "F.Cu") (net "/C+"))
 (segment (start 91.2 62.8) (end 90.6 62.2) (width 0.4) (layer "F.Cu") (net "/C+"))
 (segment (start 92.8625 63.75) (end 90.95 63.75) (width 0.4) (layer "F.Cu") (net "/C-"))
 (segment (start 90.95 63.75) (end 90.6 64.1) (width 0.4) (layer "F.Cu") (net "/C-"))
 (segment (start 94.75 67.8) (end 96.95 67.8) (width 0.4) (layer "F.Cu") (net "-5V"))
 (segment (start 94.75 71.68) (end 94.63 71.8) (width 0.4) (layer "F.Cu") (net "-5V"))
 (segment (start 98.75 63.9) (end 98.75 66) (width 0.4) (layer "F.Cu") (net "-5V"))
 (segment (start 92.09 71.8) (end 94.63 71.8) (width 0.4) (layer "F.Cu") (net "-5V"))
 (segment (start 96.95 67.8) (end 97.25 67.5) (width 0.4) (layer "F.Cu") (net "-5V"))
 (segment (start 94.75 67.8) (end 94.75 71.68) (width 0.4) (layer "F.Cu") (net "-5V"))
 (segment (start 98.75 66) (end 97.25 67.5) (width 0.4) (layer "F.Cu") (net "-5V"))
 (segment (start 105 67.9) (end 107.1 67.9) (width 0.4) (layer "F.Cu") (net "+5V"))
 (segment (start 105 69.005) (end 107.29 71.295) (width 0.4) (layer "F.Cu") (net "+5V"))
 (segment (start 105 67.9) (end 105 69.005) (width 0.4) (layer "F.Cu") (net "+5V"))
 (segment (start 107.29 71.8) (end 109.83 71.8) (width 0.4) (layer "F.Cu") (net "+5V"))
 (segment (start 107.1 67.9) (end 107.5 67.5) (width 0.4) (layer "F.Cu") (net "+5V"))
 (segment (start 107.29 71.295) (end 107.29 71.8) (width 0.4) (layer "F.Cu") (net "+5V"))
 (segment (start 109 66) (end 107.5 67.5) (width 0.4) (layer "F.Cu") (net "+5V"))
 (segment (start 109 64) (end 109 66) (width 0.4) (layer "F.Cu") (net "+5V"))
 (segment (start 107.95 53) (end 108.75 53.8) (width 0.2) (layer "F.Cu") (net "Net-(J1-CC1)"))
 (segment (start 102.63 53) (end 107.95 53) (width 0.2) (layer "F.Cu") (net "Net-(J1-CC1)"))
 (segment (start 101.375 54.855) (end 101.375 54.255) (width 0.2) (layer "F.Cu") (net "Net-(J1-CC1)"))
 (segment (start 101.375 54.255) (end 102.63 53) (width 0.2) (layer "F.Cu") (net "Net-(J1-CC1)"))
 (segment (start 100.375 54.855) (end 100.375 54.255) (width 0.2) (layer "F.Cu") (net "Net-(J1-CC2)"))
 (segment (start 100.375 54.255) (end 99.12 53) (width 0.2) (layer "F.Cu") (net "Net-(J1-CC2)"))
 (segment (start 99.12 53) (end 93.7175 53) (width 0.2) (layer "F.Cu") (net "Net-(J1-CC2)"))
 (segment (start 93.7175 53) (end 92.95 53.7675) (width 0.2) (layer "F.Cu") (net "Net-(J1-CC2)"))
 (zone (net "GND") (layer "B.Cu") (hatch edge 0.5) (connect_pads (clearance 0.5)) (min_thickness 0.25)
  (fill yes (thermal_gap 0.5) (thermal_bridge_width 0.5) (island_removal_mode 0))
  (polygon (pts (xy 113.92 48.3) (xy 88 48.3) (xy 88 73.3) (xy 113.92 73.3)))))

